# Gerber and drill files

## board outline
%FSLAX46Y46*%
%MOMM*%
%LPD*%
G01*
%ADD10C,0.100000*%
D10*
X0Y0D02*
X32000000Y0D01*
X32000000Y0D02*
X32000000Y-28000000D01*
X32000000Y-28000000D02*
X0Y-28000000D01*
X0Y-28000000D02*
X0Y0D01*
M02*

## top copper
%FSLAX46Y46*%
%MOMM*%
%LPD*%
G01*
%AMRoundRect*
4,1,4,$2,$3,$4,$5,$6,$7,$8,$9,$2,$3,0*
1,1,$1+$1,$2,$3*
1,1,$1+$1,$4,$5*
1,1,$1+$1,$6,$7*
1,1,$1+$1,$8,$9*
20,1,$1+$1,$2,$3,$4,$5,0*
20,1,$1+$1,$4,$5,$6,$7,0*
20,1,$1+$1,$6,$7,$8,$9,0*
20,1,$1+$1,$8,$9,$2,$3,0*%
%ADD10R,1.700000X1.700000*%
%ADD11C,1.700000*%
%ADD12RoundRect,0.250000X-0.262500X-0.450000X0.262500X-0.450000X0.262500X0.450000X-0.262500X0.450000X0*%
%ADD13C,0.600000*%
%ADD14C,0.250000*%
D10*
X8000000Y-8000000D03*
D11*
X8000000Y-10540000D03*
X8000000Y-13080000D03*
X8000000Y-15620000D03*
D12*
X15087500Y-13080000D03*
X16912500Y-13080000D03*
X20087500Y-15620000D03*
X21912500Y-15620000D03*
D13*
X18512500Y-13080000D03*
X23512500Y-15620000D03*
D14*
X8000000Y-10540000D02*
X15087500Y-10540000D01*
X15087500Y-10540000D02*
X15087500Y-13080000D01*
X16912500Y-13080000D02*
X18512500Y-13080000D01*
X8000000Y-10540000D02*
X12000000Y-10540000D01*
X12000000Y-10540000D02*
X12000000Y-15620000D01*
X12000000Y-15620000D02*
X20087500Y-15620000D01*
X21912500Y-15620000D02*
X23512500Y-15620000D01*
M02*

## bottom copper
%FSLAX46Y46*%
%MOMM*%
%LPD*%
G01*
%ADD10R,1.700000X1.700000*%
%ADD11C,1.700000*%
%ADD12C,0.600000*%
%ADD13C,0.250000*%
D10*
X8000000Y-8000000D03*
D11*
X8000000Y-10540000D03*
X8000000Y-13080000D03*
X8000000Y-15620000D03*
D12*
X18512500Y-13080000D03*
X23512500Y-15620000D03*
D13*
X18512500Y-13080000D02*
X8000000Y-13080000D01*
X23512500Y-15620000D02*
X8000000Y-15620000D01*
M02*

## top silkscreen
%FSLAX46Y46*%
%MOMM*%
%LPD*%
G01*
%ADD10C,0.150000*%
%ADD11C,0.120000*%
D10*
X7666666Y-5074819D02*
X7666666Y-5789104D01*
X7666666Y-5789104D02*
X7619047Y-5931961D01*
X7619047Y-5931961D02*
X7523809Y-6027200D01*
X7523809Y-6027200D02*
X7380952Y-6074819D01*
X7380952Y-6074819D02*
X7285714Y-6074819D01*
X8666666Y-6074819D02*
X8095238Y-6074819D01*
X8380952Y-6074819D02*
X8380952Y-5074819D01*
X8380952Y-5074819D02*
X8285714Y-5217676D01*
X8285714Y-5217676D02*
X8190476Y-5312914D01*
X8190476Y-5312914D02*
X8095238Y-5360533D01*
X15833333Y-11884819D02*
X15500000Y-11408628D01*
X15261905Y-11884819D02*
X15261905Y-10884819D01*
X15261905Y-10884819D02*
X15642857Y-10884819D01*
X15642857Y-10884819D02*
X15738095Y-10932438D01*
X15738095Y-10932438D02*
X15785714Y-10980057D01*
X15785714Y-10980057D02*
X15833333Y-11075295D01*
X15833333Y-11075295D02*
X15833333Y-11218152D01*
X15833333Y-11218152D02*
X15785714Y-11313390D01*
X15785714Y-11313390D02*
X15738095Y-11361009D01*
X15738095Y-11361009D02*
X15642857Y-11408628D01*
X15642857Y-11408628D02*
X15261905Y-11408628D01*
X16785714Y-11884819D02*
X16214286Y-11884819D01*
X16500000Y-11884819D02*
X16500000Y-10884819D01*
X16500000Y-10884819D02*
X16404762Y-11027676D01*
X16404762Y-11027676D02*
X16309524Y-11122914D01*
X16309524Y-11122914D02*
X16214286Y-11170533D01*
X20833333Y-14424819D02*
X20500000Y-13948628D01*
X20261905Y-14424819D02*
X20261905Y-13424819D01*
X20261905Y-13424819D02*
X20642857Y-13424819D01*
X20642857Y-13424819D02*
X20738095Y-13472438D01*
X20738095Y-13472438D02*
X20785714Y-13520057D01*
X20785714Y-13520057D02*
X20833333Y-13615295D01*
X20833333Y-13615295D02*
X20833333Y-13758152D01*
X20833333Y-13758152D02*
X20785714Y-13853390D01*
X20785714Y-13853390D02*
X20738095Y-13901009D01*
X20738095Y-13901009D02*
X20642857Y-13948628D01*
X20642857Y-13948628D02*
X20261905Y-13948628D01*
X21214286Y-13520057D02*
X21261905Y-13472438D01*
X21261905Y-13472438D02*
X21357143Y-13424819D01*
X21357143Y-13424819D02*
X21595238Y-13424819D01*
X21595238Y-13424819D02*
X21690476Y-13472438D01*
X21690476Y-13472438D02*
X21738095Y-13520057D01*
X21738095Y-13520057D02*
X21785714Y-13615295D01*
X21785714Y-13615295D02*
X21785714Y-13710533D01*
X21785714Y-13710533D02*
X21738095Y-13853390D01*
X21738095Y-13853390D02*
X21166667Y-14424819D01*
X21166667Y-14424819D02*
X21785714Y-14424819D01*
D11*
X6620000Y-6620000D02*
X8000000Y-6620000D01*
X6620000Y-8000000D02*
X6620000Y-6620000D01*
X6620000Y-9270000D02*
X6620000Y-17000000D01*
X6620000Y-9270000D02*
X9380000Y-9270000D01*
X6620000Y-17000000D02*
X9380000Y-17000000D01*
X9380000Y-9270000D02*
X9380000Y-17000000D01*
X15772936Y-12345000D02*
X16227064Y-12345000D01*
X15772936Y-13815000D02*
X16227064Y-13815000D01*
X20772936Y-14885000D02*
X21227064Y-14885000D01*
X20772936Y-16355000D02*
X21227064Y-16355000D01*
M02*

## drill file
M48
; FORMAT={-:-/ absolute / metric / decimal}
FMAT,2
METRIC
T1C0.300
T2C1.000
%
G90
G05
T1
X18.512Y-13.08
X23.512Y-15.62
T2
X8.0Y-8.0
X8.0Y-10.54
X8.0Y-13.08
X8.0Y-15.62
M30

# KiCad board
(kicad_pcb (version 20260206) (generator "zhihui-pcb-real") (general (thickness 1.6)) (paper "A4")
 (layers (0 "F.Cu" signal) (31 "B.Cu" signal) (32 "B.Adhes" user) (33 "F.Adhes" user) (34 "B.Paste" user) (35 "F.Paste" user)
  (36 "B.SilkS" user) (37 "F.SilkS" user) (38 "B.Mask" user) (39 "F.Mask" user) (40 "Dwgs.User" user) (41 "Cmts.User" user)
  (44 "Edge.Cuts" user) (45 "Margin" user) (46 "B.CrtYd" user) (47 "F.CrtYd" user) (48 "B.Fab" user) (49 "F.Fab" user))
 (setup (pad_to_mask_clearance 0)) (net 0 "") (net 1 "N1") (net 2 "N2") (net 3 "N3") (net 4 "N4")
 (gr_line (start 0 0) (end 32 0) (stroke (width 0.1) (type default)) (layer "Edge.Cuts"))
 (gr_line (start 32 0) (end 32 28) (stroke (width 0.1) (type default)) (layer "Edge.Cuts"))
 (gr_line (start 32 28) (end 0 28) (stroke (width 0.1) (type default)) (layer "Edge.Cuts"))
 (gr_line (start 0 28) (end 0 0) (stroke (width 0.1) (type default)) (layer "Edge.Cuts"))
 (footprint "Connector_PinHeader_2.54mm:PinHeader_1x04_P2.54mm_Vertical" (layer "F.Cu")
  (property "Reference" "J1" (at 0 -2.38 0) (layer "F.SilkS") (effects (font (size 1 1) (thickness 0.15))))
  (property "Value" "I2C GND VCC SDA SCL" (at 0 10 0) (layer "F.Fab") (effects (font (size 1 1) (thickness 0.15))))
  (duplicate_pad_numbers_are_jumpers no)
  (fp_line (start -1.38 -1.38) (end 0 -1.38) (stroke (width 0.12) (type solid)) (layer "F.SilkS"))
  (fp_line (start -1.38 0) (end -1.38 -1.38) (stroke (width 0.12) (type solid)) (layer "F.SilkS"))
  (fp_line (start -1.38 1.27) (end -1.38 9) (stroke (width 0.12) (type solid)) (layer "F.SilkS"))
  (fp_line (start -1.38 1.27) (end 1.38 1.27) (stroke (width 0.12) (type solid)) (layer "F.SilkS"))
  (fp_line (start -1.38 9) (end 1.38 9) (stroke (width 0.12) (type solid)) (layer "F.SilkS"))
  (fp_line (start 1.38 1.27) (end 1.38 9) (stroke (width 0.12) (type solid)) (layer "F.SilkS"))
  (pad "1" thru_hole rect (at 0 0) (size 1.7 1.7) (drill 1) (layers "*.Cu" "*.Mask") (remove_unused_layers no) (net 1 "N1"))
  (pad "2" thru_hole circle (at 0 2.54) (size 1.7 1.7) (drill 1) (layers "*.Cu" "*.Mask") (remove_unused_layers no) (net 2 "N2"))
  (pad "3" thru_hole circle (at 0 5.08) (size 1.7 1.7) (drill 1) (layers "*.Cu" "*.Mask") (remove_unused_layers no) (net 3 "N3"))
  (pad "4" thru_hole circle (at 0 7.62) (size 1.7 1.7) (drill 1) (layers "*.Cu" "*.Mask") (remove_unused_layers no) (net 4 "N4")) (at 8 8 0))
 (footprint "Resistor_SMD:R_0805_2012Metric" (layer "F.Cu")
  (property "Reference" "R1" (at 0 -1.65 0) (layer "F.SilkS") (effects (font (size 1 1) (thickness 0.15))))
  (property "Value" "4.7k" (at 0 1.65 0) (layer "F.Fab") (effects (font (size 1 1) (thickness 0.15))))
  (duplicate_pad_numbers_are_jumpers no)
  (fp_line (start -0.227064 -0.735) (end 0.227064 -0.735) (stroke (width 0.12) (type solid)) (layer "F.SilkS"))
  (fp_line (start -0.227064 0.735) (end 0.227064 0.735) (stroke (width 0.12) (type solid)) (layer "F.SilkS"))
  (pad "1" smd roundrect (at -0.9125 0) (size 1.025 1.4) (layers "F.Cu" "F.Mask" "F.Paste") (roundrect_rratio 0.243902) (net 2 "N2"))
  (pad "2" smd roundrect (at 0.9125 0) (size 1.025 1.4) (layers "F.Cu" "F.Mask" "F.Paste") (roundrect_rratio 0.243902) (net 3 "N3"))
  (at 16 13.08 0))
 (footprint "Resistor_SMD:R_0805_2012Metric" (layer "F.Cu")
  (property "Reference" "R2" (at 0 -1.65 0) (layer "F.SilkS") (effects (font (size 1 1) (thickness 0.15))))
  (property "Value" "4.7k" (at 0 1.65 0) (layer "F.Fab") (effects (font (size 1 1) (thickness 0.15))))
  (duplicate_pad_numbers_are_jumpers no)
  (fp_line (start -0.227064 -0.735) (end 0.227064 -0.735) (stroke (width 0.12) (type solid)) (layer "F.SilkS"))
  (fp_line (start -0.227064 0.735) (end 0.227064 0.735) (stroke (width 0.12) (type solid)) (layer "F.SilkS"))
  (pad "1" smd roundrect (at -0.9125 0) (size 1.025 1.4) (layers "F.Cu" "F.Mask" "F.Paste") (roundrect_rratio 0.243902) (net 2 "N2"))
  (pad "2" smd roundrect (at 0.9125 0) (size 1.025 1.4) (layers "F.Cu" "F.Mask" "F.Paste") (roundrect_rratio 0.243902) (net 4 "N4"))
  (at 21 15.62 0))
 (segment (start 8 10.54) (end 15.0875 10.54) (width 0.25) (layer "F.Cu") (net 2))
 (segment (start 15.0875 10.54) (end 15.0875 13.08) (width 0.25) (layer "F.Cu") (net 2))
 (segment (start 16.9125 13.08) (end 18.5125 13.08) (width 0.25) (layer "F.Cu") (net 3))
 (segment (start 18.5125 13.08) (end 8 13.08) (width 0.25) (layer "B.Cu") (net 3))
 (segment (start 8 10.54) (end 12 10.54) (width 0.25) (layer "F.Cu") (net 2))
 (segment (start 12 10.54) (end 12 15.62) (width 0.25) (layer "F.Cu") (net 2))
 (segment (start 12 15.62) (end 20.0875 15.62) (width 0.25) (layer "F.Cu") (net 2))
 (segment (start 21.9125 15.62) (end 23.5125 15.62) (width 0.25) (layer "F.Cu") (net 4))
 (segment (start 23.5125 15.62) (end 8 15.62) (width 0.25) (layer "B.Cu") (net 4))
 (via (at 18.5125 13.08) (size 0.6) (drill 0.3) (layers "F.Cu" "B.Cu") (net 3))
 (via (at 23.5125 15.62) (size 0.6) (drill 0.3) (layers "F.Cu" "B.Cu") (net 4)))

